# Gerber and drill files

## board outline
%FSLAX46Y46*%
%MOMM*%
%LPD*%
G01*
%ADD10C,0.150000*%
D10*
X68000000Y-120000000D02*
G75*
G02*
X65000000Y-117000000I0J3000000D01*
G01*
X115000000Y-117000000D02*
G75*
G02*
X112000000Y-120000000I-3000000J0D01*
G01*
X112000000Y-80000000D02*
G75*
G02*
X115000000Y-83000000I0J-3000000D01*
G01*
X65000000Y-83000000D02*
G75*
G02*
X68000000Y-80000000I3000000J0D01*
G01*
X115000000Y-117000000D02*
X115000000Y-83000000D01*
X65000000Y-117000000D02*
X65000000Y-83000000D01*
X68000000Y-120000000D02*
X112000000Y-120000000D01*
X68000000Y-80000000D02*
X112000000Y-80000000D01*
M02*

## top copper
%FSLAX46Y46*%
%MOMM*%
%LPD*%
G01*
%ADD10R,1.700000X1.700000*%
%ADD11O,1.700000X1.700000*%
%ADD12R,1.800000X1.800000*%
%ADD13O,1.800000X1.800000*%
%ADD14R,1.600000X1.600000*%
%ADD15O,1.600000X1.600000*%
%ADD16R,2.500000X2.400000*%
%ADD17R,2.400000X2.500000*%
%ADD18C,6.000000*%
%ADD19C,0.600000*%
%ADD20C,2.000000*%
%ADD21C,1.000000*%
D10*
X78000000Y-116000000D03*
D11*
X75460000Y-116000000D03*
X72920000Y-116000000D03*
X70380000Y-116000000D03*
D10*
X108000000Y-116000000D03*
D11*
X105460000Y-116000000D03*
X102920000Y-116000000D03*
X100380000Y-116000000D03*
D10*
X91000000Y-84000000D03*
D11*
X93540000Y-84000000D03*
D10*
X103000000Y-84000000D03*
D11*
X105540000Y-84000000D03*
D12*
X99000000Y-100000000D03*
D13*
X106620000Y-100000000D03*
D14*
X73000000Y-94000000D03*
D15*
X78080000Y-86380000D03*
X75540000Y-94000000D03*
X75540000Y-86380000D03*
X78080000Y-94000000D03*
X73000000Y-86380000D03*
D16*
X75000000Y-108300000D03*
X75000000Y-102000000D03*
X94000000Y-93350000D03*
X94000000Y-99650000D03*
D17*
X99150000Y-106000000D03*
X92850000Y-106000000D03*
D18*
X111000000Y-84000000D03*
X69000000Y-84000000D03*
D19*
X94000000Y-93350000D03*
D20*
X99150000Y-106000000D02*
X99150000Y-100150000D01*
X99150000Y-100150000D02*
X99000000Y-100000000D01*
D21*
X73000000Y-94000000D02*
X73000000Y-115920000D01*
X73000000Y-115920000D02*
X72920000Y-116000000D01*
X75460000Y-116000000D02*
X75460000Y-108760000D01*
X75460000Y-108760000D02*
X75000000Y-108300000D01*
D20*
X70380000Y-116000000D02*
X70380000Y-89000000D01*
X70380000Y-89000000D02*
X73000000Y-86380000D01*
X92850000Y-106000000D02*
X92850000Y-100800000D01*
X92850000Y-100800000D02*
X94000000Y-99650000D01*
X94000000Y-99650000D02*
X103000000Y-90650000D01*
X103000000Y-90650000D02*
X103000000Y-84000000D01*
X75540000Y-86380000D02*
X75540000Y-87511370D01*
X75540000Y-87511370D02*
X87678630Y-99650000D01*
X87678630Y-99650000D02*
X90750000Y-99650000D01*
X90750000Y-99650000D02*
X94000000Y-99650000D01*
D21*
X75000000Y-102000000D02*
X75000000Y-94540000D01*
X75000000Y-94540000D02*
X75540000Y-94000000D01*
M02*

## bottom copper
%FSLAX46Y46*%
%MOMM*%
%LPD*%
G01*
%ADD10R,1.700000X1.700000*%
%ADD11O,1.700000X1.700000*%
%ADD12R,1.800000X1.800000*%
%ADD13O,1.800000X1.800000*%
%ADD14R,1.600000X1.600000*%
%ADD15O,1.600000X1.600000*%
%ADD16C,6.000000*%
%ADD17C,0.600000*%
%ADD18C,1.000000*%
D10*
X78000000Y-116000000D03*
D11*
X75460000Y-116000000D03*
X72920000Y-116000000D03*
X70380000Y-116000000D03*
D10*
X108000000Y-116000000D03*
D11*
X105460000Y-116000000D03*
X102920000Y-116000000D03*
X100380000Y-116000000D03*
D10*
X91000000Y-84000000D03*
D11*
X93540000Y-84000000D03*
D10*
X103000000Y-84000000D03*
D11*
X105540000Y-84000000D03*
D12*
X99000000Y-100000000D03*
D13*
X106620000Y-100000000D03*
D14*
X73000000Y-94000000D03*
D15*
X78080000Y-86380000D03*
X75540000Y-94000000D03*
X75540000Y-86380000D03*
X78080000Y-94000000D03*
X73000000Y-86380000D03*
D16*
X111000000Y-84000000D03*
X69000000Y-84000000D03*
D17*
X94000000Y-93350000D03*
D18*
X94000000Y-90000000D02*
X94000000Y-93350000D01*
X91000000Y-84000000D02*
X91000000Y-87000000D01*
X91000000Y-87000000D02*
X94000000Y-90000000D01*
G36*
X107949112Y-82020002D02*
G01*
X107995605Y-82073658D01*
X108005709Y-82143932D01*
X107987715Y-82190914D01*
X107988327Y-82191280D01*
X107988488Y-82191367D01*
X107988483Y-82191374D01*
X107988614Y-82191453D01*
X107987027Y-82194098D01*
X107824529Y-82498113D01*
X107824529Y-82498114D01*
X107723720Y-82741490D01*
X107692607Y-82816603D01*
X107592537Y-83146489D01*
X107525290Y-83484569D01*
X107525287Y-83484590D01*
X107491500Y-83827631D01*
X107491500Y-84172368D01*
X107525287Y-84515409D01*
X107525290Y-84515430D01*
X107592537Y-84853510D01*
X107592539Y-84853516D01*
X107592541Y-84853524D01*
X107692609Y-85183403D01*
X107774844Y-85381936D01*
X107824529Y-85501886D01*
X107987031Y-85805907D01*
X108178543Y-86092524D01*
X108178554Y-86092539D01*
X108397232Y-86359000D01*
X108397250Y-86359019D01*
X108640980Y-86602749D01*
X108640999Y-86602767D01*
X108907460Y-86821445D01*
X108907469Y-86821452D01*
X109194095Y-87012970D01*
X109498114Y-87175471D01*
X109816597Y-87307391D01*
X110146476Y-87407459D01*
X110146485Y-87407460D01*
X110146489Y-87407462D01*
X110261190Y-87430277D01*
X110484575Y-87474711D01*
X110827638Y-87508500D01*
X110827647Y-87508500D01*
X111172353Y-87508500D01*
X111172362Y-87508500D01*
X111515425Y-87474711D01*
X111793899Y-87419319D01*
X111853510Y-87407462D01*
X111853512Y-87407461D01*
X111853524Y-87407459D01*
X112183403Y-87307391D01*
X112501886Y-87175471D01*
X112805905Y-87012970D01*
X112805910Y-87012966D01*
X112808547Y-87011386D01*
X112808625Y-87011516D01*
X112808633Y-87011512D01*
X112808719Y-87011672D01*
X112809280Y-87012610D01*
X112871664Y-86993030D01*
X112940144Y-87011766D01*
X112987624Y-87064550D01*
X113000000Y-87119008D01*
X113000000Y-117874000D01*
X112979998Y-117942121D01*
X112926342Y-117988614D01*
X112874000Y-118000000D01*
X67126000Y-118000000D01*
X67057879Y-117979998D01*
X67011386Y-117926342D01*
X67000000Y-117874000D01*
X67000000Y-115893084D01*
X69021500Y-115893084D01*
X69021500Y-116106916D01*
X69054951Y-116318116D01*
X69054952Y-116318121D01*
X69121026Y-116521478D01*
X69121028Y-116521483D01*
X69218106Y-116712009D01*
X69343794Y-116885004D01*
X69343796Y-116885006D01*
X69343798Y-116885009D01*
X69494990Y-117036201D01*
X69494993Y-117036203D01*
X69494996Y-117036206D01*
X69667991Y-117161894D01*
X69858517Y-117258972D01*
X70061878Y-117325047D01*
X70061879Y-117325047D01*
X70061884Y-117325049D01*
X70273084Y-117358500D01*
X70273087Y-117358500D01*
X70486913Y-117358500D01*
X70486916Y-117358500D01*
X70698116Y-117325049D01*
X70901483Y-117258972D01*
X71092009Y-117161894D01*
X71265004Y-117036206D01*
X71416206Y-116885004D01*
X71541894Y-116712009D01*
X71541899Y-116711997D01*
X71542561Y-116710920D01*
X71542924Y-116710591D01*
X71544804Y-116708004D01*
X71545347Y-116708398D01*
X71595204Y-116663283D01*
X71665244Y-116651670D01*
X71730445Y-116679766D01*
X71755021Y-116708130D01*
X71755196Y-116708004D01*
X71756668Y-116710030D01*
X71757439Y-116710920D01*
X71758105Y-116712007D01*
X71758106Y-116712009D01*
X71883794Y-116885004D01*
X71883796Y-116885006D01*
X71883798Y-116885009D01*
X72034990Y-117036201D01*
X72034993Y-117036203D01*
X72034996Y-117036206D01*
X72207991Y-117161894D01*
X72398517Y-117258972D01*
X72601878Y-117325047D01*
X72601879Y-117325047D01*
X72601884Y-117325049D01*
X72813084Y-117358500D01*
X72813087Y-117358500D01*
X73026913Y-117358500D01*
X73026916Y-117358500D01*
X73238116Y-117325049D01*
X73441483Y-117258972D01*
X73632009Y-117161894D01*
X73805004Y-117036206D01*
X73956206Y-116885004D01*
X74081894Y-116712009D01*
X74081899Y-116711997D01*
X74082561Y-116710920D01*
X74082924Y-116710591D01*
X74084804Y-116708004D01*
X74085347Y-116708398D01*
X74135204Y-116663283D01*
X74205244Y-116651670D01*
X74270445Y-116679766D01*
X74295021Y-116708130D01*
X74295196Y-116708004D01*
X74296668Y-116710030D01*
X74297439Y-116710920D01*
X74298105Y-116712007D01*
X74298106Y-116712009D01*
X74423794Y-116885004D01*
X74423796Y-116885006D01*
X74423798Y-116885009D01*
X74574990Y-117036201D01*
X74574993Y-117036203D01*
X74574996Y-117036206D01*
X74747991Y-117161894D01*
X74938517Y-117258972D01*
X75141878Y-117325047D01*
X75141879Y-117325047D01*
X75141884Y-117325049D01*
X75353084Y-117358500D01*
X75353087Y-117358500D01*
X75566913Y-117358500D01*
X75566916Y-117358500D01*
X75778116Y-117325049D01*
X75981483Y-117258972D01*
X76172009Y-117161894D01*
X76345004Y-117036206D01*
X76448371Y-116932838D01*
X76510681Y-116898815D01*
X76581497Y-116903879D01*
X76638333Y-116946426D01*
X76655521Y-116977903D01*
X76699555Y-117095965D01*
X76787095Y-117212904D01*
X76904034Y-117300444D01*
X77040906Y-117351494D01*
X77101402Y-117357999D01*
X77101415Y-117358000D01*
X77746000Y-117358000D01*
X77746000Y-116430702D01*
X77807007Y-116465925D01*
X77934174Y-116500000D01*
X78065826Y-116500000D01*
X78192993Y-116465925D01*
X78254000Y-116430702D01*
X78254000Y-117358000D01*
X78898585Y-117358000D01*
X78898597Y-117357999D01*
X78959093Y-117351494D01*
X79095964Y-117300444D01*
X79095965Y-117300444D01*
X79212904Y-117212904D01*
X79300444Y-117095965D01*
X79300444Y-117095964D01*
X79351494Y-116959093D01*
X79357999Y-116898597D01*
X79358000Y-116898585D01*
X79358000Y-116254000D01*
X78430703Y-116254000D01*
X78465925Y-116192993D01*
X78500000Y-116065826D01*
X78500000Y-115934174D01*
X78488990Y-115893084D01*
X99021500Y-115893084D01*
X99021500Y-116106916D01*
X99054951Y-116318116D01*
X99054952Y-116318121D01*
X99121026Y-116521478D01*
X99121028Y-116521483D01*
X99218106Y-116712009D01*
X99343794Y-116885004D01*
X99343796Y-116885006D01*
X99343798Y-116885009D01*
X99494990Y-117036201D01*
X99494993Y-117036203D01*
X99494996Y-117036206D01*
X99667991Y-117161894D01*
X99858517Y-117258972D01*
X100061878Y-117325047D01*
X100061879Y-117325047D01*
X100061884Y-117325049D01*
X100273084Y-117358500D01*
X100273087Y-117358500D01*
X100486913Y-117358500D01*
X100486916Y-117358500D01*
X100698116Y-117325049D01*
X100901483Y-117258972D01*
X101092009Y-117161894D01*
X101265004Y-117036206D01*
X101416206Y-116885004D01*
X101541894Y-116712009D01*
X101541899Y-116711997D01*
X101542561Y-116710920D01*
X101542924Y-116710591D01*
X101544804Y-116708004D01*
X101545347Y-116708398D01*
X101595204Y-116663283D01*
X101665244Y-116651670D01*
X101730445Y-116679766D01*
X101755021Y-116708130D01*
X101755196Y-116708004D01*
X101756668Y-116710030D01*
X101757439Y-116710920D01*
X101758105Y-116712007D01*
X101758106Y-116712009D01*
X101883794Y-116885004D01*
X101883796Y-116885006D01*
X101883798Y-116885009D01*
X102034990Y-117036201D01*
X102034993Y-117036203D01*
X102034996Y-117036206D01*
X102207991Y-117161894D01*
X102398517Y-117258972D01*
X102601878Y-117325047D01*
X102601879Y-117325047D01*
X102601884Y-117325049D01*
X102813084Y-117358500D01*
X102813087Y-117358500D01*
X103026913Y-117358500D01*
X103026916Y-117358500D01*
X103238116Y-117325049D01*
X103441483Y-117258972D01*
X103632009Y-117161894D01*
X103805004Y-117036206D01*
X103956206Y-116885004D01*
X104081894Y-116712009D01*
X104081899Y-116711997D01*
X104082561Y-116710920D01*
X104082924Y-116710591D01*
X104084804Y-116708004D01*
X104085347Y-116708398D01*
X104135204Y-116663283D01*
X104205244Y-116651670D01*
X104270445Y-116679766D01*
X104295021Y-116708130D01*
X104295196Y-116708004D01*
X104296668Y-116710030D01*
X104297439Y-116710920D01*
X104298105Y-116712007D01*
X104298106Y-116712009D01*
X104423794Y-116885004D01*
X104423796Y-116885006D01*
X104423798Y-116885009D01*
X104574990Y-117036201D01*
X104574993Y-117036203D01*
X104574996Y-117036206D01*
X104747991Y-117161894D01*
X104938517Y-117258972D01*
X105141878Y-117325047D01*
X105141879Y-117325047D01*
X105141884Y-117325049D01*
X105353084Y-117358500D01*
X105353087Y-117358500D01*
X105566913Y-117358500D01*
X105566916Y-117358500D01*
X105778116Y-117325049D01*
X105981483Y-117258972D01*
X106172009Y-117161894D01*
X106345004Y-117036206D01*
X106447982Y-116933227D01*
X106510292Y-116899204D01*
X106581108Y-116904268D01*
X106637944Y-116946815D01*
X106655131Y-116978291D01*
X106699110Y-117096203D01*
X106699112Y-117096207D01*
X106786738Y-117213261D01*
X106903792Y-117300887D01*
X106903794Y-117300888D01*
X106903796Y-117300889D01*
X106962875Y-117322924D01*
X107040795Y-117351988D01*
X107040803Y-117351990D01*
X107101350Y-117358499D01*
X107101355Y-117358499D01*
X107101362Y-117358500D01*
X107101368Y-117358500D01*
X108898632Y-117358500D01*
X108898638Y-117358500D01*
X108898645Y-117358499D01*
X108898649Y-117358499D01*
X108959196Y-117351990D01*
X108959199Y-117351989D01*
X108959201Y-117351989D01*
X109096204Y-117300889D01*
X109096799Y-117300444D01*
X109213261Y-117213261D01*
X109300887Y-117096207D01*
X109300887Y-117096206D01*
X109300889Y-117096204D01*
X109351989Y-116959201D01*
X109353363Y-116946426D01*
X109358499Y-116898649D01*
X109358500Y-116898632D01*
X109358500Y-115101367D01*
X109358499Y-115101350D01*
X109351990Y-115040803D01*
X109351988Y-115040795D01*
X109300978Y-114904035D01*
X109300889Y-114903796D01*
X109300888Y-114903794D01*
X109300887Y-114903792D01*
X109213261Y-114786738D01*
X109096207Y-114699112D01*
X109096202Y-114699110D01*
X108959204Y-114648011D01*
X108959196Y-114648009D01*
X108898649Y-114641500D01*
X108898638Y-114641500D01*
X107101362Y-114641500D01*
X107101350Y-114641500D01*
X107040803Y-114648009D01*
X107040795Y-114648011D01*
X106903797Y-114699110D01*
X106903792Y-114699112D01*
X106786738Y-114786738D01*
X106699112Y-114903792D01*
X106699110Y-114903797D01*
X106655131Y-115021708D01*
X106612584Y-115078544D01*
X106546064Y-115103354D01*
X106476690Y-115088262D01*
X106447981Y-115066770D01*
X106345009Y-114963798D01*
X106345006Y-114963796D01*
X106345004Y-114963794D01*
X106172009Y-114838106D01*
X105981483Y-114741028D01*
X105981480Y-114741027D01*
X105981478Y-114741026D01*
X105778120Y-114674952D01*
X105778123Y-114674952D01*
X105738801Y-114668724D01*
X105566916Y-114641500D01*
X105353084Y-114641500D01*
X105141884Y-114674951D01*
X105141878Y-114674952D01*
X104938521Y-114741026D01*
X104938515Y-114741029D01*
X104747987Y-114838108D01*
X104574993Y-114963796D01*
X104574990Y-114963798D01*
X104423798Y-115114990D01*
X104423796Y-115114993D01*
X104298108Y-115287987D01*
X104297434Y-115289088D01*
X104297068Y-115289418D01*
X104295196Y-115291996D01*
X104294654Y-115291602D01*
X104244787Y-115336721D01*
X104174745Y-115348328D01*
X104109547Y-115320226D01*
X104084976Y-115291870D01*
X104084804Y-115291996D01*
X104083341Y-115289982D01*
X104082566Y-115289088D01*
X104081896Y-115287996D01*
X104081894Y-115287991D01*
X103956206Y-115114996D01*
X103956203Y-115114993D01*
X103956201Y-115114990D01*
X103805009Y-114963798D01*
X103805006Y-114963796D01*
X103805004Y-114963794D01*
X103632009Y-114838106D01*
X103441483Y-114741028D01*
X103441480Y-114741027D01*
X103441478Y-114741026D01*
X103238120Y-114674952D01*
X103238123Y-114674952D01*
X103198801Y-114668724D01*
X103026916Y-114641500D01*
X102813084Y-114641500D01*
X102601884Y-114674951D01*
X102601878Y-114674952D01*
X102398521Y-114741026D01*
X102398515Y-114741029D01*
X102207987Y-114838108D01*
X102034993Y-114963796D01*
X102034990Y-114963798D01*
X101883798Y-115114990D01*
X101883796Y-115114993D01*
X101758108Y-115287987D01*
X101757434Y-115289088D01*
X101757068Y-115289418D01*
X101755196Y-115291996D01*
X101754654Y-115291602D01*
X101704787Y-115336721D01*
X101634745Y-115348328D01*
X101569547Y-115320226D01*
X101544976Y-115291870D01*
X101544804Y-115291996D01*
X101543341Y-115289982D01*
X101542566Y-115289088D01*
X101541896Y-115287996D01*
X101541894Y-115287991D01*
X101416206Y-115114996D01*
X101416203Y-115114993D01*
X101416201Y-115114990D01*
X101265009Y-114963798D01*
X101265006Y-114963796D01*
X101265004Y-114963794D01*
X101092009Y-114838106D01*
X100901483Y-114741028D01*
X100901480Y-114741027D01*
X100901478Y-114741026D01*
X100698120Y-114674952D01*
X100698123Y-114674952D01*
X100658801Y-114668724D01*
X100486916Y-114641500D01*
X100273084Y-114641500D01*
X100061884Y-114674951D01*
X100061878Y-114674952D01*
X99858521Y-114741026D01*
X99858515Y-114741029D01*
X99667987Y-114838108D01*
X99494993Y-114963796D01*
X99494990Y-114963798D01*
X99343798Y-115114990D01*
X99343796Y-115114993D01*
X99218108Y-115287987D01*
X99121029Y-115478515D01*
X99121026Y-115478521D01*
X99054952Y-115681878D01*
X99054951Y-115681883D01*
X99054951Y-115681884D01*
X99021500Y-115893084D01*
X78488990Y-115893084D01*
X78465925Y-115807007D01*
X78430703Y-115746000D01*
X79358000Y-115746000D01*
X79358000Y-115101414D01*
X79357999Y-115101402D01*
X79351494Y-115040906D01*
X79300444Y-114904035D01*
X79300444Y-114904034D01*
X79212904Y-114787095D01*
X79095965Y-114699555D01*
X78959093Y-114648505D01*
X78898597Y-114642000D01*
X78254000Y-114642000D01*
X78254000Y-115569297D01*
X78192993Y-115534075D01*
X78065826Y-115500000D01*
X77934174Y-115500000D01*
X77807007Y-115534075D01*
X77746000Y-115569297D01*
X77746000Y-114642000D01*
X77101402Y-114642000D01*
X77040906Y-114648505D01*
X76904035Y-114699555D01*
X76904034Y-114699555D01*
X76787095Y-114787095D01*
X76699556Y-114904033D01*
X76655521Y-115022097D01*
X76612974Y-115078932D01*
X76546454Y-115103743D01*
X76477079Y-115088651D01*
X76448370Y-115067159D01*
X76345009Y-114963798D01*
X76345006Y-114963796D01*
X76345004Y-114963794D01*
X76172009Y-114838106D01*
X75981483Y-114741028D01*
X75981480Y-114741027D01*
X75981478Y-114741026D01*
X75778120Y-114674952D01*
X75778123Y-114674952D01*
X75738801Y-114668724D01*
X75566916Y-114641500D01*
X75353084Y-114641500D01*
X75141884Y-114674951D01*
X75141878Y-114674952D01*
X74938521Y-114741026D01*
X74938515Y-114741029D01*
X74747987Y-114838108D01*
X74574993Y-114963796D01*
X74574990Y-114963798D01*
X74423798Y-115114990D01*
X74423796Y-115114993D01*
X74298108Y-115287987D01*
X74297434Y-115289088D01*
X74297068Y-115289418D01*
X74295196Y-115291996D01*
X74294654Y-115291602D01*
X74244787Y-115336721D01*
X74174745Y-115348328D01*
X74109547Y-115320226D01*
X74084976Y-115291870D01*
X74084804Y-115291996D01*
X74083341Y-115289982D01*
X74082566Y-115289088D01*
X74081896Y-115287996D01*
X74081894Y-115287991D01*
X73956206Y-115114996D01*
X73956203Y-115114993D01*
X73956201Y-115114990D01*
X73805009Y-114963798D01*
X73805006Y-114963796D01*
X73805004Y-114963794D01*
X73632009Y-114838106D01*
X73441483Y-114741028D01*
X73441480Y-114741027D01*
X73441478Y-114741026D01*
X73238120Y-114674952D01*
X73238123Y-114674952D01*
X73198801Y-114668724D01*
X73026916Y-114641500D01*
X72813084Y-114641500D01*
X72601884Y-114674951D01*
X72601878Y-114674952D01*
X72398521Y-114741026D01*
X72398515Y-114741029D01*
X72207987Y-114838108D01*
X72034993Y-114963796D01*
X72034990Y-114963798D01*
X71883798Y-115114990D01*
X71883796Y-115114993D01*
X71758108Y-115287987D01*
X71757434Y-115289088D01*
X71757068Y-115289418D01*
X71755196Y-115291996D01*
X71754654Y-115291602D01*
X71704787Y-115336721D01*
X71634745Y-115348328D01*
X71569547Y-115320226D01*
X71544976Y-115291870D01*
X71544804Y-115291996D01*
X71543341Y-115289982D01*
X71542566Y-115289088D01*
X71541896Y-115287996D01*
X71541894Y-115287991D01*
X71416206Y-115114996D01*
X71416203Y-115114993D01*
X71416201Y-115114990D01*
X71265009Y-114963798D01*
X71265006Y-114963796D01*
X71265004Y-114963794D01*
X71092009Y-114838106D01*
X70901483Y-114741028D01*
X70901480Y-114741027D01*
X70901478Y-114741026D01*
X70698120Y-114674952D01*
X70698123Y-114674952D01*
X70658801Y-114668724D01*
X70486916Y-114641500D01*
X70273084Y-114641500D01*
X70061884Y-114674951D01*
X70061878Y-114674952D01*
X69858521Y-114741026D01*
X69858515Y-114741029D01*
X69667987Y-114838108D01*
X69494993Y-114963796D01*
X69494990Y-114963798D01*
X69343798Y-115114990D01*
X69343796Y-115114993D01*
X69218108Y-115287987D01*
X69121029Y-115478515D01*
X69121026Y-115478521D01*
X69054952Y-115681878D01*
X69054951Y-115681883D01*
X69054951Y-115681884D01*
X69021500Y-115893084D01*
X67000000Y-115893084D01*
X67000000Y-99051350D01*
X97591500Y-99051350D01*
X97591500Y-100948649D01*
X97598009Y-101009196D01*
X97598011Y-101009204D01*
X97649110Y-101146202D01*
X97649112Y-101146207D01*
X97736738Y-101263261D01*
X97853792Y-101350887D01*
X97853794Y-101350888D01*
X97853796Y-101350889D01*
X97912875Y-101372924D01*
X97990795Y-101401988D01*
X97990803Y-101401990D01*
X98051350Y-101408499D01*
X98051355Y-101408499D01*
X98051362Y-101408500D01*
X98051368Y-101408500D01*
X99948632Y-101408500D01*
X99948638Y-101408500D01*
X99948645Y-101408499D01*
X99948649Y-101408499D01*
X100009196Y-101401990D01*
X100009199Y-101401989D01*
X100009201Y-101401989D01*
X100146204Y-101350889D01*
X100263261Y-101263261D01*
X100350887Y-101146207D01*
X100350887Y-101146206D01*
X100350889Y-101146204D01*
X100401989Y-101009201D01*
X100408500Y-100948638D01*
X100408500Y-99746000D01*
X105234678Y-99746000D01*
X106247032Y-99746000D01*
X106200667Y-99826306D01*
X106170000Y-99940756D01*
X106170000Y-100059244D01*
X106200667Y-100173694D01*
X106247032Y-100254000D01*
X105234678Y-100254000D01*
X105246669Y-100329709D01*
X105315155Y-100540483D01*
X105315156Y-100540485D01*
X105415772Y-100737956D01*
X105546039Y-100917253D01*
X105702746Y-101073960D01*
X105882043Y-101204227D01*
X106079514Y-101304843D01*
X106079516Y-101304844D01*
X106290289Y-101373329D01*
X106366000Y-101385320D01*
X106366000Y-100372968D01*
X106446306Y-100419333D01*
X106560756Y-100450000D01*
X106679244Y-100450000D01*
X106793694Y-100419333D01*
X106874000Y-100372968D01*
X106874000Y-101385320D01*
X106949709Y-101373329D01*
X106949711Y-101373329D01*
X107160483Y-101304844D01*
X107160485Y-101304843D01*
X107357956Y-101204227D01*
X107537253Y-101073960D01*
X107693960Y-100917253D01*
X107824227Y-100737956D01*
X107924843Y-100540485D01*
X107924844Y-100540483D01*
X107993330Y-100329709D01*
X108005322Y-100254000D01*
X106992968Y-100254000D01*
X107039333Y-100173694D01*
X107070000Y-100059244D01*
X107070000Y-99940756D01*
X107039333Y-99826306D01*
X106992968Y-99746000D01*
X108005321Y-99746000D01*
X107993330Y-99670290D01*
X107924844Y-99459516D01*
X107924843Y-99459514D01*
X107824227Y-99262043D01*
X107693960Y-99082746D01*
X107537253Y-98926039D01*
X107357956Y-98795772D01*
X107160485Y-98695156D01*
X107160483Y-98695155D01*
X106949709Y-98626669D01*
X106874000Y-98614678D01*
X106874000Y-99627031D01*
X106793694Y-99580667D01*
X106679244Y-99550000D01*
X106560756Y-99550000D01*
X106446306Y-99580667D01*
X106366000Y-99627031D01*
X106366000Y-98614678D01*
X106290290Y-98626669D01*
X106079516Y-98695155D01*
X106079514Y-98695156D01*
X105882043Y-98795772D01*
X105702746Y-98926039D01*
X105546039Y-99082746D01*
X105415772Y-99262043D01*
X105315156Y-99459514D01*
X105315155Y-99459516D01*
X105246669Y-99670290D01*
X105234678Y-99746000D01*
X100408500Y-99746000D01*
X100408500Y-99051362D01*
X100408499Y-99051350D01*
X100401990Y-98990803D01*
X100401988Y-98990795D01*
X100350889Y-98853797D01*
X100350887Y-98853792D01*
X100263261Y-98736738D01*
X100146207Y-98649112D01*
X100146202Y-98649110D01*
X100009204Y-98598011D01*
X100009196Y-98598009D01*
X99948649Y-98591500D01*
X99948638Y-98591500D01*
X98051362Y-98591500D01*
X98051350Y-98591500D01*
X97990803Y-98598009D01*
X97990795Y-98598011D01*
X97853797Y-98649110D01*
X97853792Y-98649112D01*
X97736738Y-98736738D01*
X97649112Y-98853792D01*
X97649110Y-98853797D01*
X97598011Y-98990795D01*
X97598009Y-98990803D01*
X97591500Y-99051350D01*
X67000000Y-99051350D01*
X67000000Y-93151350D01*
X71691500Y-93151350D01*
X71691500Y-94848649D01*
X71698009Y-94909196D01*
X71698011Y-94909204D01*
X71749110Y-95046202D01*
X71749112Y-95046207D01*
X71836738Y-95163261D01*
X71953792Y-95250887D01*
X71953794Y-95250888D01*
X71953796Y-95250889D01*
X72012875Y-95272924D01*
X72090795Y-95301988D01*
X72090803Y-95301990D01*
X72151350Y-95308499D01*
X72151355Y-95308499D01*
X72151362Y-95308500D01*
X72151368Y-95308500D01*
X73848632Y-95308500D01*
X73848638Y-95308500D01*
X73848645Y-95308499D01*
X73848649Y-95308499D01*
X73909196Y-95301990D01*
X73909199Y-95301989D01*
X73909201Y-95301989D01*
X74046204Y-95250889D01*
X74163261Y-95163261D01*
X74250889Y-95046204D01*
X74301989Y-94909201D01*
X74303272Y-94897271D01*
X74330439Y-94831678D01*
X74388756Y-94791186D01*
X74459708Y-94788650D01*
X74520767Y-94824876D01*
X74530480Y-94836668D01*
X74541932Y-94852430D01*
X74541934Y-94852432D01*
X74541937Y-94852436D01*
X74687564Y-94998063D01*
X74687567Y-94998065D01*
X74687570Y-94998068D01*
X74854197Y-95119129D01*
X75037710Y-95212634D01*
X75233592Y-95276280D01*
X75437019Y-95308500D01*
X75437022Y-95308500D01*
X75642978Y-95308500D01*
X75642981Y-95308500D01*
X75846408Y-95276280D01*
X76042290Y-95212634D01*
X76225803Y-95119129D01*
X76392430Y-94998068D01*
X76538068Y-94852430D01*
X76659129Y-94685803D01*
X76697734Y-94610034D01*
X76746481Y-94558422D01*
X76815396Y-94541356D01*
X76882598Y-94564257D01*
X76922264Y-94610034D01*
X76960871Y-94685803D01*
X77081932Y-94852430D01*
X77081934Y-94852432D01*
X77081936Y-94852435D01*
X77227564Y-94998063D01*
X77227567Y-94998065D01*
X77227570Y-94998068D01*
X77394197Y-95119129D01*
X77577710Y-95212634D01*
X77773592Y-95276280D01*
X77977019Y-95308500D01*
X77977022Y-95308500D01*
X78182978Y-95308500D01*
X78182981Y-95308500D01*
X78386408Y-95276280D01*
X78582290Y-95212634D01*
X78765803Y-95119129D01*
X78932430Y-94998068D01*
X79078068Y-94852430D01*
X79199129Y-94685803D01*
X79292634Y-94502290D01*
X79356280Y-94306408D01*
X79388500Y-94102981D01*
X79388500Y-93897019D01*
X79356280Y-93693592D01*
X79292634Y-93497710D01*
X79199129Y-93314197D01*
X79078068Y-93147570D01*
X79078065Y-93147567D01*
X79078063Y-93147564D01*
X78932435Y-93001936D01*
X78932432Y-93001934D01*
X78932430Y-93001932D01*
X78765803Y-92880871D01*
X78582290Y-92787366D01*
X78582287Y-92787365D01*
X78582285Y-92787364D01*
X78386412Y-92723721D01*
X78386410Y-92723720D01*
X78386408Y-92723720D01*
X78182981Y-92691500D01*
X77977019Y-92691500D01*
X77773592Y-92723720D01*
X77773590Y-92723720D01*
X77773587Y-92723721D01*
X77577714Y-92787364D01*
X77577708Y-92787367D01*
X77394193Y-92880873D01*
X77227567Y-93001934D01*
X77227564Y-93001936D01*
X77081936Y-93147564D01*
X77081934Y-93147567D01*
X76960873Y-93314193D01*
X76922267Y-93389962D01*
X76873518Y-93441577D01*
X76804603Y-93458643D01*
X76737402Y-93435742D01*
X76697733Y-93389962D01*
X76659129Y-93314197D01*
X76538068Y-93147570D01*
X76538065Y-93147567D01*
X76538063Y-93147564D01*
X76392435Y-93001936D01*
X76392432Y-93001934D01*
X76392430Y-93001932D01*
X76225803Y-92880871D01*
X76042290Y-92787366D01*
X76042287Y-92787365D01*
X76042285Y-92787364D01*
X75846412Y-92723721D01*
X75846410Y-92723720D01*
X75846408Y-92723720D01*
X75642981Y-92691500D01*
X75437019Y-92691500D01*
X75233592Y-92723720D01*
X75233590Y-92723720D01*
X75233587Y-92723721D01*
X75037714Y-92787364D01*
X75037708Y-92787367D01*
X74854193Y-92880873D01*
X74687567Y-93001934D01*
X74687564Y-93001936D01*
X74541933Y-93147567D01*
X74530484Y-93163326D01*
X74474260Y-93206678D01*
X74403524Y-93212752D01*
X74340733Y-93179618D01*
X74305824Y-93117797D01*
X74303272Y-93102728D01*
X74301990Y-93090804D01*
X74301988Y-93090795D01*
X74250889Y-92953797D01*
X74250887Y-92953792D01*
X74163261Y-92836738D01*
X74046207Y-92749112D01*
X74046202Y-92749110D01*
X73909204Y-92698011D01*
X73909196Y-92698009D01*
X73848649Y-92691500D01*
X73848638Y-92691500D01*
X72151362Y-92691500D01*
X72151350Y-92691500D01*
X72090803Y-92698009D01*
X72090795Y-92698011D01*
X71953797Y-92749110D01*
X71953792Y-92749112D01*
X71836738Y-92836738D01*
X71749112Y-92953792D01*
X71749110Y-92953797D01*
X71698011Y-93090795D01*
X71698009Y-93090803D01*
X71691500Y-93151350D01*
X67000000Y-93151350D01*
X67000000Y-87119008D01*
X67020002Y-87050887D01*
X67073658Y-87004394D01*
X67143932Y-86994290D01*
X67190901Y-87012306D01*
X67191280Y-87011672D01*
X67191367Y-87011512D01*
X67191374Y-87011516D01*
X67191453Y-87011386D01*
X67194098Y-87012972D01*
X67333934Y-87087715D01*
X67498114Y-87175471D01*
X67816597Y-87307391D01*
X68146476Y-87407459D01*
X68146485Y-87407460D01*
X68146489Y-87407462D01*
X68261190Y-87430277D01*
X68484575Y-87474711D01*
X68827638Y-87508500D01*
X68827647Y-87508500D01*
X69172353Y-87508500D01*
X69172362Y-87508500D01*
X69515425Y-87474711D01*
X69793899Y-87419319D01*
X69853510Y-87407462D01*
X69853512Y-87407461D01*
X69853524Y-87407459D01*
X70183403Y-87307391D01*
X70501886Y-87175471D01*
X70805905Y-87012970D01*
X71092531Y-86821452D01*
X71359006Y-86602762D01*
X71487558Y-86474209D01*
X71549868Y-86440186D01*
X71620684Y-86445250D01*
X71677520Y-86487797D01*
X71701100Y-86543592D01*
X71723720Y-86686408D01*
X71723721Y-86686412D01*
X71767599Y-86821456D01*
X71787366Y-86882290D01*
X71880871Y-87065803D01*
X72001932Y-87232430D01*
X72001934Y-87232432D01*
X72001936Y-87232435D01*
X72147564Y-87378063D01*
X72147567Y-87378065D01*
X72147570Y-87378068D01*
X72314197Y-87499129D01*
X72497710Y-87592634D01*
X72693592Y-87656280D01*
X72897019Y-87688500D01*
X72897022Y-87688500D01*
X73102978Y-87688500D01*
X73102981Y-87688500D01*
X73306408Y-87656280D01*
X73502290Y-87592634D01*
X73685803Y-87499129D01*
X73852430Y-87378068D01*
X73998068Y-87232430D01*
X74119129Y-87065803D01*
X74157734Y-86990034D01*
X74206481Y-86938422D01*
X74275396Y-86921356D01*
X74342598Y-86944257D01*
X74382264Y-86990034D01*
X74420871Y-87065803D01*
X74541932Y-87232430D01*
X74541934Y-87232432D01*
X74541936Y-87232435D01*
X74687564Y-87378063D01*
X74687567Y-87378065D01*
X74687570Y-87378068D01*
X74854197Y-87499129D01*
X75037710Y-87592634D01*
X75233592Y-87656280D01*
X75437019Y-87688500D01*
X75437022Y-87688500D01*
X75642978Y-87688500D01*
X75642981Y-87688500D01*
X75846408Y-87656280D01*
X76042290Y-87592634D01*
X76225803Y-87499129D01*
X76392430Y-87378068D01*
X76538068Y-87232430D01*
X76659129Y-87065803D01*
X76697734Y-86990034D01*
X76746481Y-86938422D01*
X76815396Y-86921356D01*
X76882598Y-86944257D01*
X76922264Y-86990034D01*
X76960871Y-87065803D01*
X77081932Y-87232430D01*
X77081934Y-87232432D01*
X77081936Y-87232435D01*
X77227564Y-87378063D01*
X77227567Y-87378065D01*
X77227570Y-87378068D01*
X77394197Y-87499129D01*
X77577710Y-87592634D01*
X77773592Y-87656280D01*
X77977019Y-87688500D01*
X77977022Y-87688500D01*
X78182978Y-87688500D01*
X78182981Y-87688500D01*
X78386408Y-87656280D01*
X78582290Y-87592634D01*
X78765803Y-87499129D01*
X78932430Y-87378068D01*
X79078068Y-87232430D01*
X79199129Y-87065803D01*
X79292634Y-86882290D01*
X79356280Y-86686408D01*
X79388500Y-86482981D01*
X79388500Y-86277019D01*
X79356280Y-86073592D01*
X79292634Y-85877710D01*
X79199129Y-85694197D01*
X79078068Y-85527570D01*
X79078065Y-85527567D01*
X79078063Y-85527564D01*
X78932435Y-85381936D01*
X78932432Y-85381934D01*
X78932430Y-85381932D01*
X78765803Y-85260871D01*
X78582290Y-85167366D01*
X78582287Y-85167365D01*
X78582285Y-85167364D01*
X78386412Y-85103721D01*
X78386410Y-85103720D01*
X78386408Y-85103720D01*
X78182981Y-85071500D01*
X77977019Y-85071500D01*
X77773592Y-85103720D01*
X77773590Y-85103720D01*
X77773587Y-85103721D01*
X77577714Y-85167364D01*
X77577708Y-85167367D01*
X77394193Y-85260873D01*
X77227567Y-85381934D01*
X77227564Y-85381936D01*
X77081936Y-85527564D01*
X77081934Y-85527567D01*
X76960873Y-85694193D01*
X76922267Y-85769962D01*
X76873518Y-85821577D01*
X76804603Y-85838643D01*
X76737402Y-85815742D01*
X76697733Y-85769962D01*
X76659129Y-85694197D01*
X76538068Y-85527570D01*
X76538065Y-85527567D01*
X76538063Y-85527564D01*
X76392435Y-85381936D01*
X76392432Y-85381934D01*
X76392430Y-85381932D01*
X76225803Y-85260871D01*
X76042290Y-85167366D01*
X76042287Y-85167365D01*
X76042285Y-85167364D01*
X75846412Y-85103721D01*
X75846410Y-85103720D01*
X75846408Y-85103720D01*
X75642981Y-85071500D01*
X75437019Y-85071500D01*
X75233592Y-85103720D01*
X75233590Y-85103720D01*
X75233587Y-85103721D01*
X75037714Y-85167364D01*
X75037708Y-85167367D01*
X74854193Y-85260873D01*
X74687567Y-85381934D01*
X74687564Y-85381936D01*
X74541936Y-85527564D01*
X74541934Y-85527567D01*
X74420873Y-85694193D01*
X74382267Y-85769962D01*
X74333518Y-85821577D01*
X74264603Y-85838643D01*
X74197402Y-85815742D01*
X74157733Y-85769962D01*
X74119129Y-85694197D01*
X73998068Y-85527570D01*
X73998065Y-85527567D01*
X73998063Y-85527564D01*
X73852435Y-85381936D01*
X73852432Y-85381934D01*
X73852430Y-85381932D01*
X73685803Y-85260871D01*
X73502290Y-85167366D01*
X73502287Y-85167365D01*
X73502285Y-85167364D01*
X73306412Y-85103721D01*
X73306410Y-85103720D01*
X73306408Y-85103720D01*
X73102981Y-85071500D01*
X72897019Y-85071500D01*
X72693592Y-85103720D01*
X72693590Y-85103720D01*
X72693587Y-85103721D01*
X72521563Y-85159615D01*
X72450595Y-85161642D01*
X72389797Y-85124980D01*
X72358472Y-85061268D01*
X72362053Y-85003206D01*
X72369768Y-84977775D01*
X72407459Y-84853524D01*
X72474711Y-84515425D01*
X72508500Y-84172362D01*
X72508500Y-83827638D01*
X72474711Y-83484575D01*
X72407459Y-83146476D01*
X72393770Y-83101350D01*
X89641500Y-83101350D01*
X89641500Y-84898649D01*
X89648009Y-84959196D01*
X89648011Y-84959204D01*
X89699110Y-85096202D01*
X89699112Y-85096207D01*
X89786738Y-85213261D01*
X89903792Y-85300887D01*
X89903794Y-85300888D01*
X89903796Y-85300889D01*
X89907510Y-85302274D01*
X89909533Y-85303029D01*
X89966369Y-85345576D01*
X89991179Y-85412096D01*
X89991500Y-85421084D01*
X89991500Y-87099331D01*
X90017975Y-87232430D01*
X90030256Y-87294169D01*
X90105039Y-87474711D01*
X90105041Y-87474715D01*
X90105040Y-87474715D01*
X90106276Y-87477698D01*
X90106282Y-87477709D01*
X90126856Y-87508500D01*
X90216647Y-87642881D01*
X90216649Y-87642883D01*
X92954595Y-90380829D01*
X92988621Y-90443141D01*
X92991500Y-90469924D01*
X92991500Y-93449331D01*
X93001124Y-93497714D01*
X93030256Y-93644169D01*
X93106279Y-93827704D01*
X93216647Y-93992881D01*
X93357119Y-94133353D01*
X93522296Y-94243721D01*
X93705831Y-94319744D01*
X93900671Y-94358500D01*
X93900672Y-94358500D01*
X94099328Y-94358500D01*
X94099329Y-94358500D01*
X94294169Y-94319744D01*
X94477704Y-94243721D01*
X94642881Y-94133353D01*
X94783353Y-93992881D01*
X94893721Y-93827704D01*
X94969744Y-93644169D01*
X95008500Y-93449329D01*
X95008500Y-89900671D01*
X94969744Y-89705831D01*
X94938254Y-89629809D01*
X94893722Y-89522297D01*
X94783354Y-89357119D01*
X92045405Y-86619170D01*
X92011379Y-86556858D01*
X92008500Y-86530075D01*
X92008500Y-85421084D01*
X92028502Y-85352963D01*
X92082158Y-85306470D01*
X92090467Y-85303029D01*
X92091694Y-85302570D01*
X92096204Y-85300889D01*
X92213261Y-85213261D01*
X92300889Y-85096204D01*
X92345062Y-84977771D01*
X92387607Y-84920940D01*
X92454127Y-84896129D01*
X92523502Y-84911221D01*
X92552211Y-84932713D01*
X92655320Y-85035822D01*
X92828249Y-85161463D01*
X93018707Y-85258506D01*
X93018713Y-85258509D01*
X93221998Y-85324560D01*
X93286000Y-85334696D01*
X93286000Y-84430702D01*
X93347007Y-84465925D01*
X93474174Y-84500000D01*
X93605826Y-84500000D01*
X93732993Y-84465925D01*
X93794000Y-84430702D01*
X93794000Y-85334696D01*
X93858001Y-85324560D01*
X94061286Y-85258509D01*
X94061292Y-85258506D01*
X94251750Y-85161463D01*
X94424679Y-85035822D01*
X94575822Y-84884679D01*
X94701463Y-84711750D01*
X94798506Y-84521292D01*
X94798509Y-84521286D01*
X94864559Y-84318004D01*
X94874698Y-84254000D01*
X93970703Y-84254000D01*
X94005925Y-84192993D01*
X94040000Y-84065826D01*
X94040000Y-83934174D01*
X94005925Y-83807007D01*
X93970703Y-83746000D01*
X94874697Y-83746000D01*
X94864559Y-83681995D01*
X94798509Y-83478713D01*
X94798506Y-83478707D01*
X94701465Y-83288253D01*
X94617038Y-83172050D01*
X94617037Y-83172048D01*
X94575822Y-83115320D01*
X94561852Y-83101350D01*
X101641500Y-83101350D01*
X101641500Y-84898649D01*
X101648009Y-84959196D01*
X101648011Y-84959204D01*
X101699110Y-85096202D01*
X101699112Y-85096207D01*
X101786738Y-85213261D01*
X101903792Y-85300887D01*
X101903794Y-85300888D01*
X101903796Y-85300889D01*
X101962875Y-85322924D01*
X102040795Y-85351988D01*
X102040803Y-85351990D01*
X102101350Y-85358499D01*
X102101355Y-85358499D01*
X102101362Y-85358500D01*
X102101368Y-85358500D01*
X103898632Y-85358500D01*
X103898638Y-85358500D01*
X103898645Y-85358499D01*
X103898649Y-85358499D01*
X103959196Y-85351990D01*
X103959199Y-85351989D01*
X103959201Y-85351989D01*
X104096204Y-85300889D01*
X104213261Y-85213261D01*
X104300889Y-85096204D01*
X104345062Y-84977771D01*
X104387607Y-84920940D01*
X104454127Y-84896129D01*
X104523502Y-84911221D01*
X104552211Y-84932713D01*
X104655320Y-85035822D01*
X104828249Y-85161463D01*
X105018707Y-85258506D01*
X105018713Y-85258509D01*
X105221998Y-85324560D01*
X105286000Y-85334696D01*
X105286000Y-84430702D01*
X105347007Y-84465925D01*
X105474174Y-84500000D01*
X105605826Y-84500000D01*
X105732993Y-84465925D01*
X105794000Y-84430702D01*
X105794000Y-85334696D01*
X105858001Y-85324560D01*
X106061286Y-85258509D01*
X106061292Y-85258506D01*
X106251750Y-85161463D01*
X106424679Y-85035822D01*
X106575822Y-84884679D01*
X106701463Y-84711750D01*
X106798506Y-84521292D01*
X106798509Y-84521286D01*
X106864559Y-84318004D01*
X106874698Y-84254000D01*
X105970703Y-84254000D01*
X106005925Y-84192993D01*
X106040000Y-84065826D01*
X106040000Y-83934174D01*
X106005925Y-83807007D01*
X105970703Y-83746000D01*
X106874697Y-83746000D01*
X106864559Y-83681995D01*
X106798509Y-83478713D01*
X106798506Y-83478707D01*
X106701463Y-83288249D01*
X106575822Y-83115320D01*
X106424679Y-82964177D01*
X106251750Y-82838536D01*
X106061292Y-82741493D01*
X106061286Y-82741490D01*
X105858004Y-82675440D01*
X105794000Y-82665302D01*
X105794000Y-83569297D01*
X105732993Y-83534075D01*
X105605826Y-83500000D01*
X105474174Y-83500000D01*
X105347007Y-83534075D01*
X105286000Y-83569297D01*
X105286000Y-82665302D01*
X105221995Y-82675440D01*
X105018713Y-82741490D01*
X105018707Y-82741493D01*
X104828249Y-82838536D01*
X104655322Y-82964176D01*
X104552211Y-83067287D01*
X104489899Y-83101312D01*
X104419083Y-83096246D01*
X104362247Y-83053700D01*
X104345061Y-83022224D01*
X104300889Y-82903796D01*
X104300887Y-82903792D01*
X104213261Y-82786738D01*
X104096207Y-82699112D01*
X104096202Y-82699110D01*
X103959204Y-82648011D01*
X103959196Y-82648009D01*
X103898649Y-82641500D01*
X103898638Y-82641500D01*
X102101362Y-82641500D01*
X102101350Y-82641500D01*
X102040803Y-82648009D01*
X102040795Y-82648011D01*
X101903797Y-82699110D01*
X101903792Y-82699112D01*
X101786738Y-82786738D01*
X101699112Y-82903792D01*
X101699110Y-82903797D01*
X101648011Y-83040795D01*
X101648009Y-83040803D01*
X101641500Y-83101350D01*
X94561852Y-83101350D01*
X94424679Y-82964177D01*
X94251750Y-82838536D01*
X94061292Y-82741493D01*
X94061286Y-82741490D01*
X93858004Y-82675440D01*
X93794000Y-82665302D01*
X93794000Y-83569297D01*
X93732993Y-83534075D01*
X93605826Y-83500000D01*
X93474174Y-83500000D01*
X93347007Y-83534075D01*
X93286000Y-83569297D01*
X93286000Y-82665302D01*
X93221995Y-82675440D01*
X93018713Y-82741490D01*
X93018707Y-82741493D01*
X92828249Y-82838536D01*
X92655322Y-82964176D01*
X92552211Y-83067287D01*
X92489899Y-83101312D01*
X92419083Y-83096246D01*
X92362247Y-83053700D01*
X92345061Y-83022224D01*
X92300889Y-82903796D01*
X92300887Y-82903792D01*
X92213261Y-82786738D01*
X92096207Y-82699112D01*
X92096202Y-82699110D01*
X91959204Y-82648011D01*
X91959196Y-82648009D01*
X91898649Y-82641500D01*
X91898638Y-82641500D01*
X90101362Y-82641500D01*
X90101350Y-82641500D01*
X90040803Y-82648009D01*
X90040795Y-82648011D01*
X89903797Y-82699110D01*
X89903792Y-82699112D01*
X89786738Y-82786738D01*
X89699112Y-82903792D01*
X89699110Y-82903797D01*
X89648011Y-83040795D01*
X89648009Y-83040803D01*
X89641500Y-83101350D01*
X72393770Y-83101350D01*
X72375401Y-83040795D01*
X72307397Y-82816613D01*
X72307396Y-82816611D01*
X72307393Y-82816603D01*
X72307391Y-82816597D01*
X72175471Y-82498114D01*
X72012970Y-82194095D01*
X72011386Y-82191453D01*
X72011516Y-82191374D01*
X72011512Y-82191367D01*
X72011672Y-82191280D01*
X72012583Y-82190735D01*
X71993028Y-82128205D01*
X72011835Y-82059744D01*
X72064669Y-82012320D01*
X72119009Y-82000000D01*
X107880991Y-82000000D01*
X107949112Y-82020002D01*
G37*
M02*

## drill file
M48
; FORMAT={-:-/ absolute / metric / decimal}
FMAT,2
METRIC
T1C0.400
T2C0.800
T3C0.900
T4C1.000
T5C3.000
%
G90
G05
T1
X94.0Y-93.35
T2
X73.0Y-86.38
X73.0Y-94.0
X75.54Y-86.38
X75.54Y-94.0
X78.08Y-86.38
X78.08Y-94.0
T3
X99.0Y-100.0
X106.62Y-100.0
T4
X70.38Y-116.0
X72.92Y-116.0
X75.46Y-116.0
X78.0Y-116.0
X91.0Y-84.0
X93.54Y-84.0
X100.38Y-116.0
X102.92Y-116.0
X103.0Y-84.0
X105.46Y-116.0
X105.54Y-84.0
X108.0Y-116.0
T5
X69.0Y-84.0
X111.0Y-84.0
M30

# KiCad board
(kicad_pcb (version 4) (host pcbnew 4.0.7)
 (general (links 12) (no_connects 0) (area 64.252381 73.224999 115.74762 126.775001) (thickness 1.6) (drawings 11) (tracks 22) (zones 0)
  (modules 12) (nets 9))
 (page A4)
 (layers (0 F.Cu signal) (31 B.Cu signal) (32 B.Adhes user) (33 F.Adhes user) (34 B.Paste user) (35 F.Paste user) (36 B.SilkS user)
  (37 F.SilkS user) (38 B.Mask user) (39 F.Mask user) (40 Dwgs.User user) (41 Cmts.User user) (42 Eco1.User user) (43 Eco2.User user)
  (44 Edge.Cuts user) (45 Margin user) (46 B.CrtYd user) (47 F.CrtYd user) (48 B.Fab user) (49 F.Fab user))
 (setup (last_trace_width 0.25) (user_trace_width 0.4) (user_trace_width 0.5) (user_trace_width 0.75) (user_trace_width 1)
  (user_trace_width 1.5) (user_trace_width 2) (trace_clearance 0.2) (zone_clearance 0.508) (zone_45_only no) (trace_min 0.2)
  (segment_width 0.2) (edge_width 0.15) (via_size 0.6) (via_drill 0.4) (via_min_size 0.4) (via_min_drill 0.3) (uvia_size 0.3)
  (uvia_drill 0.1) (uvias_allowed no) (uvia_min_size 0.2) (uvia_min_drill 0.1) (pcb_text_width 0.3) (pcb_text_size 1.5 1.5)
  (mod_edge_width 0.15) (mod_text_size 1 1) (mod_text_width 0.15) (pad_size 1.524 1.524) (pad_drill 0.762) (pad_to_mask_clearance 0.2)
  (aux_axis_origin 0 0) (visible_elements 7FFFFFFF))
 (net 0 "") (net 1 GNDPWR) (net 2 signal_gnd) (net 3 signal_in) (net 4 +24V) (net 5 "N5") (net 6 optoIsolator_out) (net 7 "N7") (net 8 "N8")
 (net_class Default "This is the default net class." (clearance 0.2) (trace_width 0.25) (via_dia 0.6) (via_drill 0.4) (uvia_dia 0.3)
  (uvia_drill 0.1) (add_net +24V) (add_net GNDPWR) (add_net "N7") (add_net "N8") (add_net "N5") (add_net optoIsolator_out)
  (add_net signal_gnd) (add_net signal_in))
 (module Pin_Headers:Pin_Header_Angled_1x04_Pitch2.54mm (layer F.Cu) (at 78 116 270)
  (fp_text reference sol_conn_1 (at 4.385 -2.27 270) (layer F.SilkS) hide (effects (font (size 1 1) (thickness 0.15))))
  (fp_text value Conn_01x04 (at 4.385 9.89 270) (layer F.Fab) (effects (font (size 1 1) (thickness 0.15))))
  (pad 1 thru_hole rect (at 0 0 270) (size 1.7 1.7) (drill 1) (layers *.Cu *.Mask) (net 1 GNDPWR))
  (pad 2 thru_hole oval (at 0 2.54 270) (size 1.7 1.7) (drill 1) (layers *.Cu *.Mask) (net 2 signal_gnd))
  (pad 3 thru_hole oval (at 0 5.08 270) (size 1.7 1.7) (drill 1) (layers *.Cu *.Mask) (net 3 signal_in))
  (pad 4 thru_hole oval (at 0 7.62 270) (size 1.7 1.7) (drill 1) (layers *.Cu *.Mask) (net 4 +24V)))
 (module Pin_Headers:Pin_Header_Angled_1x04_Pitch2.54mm (layer F.Cu) (at 108 116 270)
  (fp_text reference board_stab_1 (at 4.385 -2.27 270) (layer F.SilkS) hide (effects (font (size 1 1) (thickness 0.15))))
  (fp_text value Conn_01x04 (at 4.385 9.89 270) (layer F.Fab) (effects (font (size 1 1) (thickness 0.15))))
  (pad 1 thru_hole rect (at 0 0 270) (size 1.7 1.7) (drill 1) (layers *.Cu *.Mask))
  (pad 2 thru_hole oval (at 0 2.54 270) (size 1.7 1.7) (drill 1) (layers *.Cu *.Mask))
  (pad 3 thru_hole oval (at 0 5.08 270) (size 1.7 1.7) (drill 1) (layers *.Cu *.Mask))
  (pad 4 thru_hole oval (at 0 7.62 270) (size 1.7 1.7) (drill 1) (layers *.Cu *.Mask)))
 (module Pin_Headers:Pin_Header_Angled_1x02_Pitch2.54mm (layer F.Cu) (at 91 84 90)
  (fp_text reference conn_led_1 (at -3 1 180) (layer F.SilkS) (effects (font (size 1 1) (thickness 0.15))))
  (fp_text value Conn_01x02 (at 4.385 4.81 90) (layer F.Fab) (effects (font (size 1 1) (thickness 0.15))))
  (pad 1 thru_hole rect (at 0 0 90) (size 1.7 1.7) (drill 1) (layers *.Cu *.Mask) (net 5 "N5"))
  (pad 2 thru_hole oval (at 0 2.54 90) (size 1.7 1.7) (drill 1) (layers *.Cu *.Mask) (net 1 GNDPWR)))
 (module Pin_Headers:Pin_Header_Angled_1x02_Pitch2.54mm (layer F.Cu) (at 103 84 90)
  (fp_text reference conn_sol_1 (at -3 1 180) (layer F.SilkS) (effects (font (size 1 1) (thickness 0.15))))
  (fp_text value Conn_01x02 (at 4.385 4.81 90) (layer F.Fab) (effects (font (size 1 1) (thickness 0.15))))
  (pad 1 thru_hole rect (at 0 0 90) (size 1.7 1.7) (drill 1) (layers *.Cu *.Mask) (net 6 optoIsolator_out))
  (pad 2 thru_hole oval (at 0 2.54 90) (size 1.7 1.7) (drill 1) (layers *.Cu *.Mask) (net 1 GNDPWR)))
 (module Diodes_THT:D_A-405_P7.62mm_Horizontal (layer F.Cu) (at 99 100)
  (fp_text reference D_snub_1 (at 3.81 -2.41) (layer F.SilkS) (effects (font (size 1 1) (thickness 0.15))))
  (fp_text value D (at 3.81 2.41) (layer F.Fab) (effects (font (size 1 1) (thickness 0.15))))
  (pad 1 thru_hole rect (at 0 0) (size 1.8 1.8) (drill 0.9) (layers *.Cu *.Mask) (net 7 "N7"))
  (pad 2 thru_hole oval (at 7.62 0) (size 1.8 1.8) (drill 0.9) (layers *.Cu *.Mask) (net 1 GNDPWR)))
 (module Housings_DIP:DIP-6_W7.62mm (layer F.Cu) (at 73 94 90)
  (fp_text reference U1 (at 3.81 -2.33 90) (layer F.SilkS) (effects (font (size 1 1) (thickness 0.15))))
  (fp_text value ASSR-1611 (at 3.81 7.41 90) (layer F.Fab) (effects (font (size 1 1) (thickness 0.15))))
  (pad 1 thru_hole rect (at 0 0 90) (size 1.6 1.6) (drill 0.8) (layers *.Cu *.Mask) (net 3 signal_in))
  (pad 4 thru_hole oval (at 7.62 5.08 90) (size 1.6 1.6) (drill 0.8) (layers *.Cu *.Mask))
  (pad 2 thru_hole oval (at 0 2.54 90) (size 1.6 1.6) (drill 0.8) (layers *.Cu *.Mask) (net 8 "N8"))
  (pad 5 thru_hole oval (at 7.62 2.54 90) (size 1.6 1.6) (drill 0.8) (layers *.Cu *.Mask) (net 6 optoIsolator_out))
  (pad 3 thru_hole oval (at 0 5.08 90) (size 1.6 1.6) (drill 0.8) (layers *.Cu *.Mask))
  (pad 6 thru_hole oval (at 7.62 0 90) (size 1.6 1.6) (drill 0.8) (layers *.Cu *.Mask) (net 4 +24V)))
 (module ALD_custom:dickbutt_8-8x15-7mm (layer F.Cu) (at 81 103.5)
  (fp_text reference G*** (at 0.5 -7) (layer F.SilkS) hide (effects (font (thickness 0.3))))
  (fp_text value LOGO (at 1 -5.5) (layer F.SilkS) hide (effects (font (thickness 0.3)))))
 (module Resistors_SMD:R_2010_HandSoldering (layer F.Cu) (at 75 105.15 90)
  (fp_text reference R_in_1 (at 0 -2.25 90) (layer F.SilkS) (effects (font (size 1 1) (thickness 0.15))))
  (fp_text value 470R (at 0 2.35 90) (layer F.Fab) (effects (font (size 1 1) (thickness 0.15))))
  (pad 1 smd rect (at -3.15 0 90) (size 2.4 2.5) (layers F.Cu F.Paste F.Mask) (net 2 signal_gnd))
  (pad 2 smd rect (at 3.15 0 90) (size 2.4 2.5) (layers F.Cu F.Paste F.Mask) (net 8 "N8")))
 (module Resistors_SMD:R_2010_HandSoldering (layer F.Cu) (at 94 96.5 270)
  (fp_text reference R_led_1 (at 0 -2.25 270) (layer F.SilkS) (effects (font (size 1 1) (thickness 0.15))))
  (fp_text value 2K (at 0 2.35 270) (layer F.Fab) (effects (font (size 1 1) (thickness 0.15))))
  (pad 1 smd rect (at -3.15 0 270) (size 2.4 2.5) (layers F.Cu F.Paste F.Mask) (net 5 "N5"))
  (pad 2 smd rect (at 3.15 0 270) (size 2.4 2.5) (layers F.Cu F.Paste F.Mask) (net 6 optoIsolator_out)))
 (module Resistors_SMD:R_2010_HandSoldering (layer F.Cu) (at 96 106 180)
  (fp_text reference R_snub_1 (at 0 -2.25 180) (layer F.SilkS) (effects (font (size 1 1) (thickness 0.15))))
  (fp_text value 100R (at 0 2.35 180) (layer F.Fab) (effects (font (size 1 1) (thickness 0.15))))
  (pad 1 smd rect (at -3.15 0 180) (size 2.4 2.5) (layers F.Cu F.Paste F.Mask) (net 7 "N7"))
  (pad 2 smd rect (at 3.15 0 180) (size 2.4 2.5) (layers F.Cu F.Paste F.Mask) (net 6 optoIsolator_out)))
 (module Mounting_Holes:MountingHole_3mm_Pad (layer F.Cu) (at 111 84)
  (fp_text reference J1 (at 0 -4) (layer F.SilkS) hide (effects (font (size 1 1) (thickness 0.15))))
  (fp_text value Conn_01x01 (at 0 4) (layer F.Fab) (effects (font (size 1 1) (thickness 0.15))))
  (pad 1 thru_hole circle (at 0 0) (size 6 6) (drill 3) (layers *.Cu *.Mask)))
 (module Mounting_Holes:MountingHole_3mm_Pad (layer F.Cu) (at 69 84)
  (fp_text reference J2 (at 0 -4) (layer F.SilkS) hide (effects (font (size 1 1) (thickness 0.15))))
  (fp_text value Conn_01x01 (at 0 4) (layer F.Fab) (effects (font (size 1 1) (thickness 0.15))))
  (pad 1 thru_hole circle (at 0 0) (size 6 6) (drill 3) (layers *.Cu *.Mask)))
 (gr_arc (start 68 117) (end 68 120) (angle 90) (layer Edge.Cuts) (width 0.15))
 (gr_arc (start 112 117) (end 115 117) (angle 90) (layer Edge.Cuts) (width 0.15))
 (gr_arc (start 112 83) (end 112 80) (angle 90) (layer Edge.Cuts) (width 0.15))
 (gr_arc (start 68 83) (end 65 83) (angle 90) (layer Edge.Cuts) (width 0.15))
 (gr_line (start 115 117) (end 115 83) (angle 90) (layer Edge.Cuts) (width 0.15))
 (gr_line (start 65 117) (end 65 83) (angle 90) (layer Edge.Cuts) (width 0.15))
 (gr_line (start 68 120) (end 112 120) (angle 90) (layer Edge.Cuts) (width 0.15))
 (gr_line (start 68 80) (end 112 80) (angle 90) (layer Edge.Cuts) (width 0.15))
 (segment (start 94 90) (end 94 93.35) (width 1) (layer B.Cu) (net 5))
 (via (at 94 93.35) (size 0.6) (drill 0.4) (layers F.Cu B.Cu) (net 5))
 (segment (start 91 84) (end 91 87) (width 1) (layer B.Cu) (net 5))
 (segment (start 91 87) (end 94 90) (width 1) (layer B.Cu) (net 5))
 (segment (start 99.15 106) (end 99.15 100.15) (width 2) (layer F.Cu) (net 7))
 (segment (start 99.15 100.15) (end 99 100) (width 2) (layer F.Cu) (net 7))
 (segment (start 73 94) (end 73 115.92) (width 1) (layer F.Cu) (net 3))
 (segment (start 73 115.92) (end 72.92 116) (width 1) (layer F.Cu) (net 3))
 (segment (start 75.46 116) (end 75.46 108.76) (width 1) (layer F.Cu) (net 2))
 (segment (start 75.46 108.76) (end 75 108.3) (width 1) (layer F.Cu) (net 2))
 (segment (start 70.38 116) (end 70.38 89) (width 2) (layer F.Cu) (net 4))
 (segment (start 70.38 89) (end 73 86.38) (width 2) (layer F.Cu) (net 4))
 (segment (start 92.85 106) (end 92.85 100.8) (width 2) (layer F.Cu) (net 6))
 (segment (start 92.85 100.8) (end 94 99.65) (width 2) (layer F.Cu) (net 6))
 (segment (start 94 99.65) (end 103 90.65) (width 2) (layer F.Cu) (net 6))
 (segment (start 103 90.65) (end 103 84) (width 2) (layer F.Cu) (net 6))
 (segment (start 75.54 86.38) (end 75.54 87.51137) (width 2) (layer F.Cu) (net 6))
 (segment (start 75.54 87.51137) (end 87.67863 99.65) (width 2) (layer F.Cu) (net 6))
 (segment (start 87.67863 99.65) (end 90.75 99.65) (width 2) (layer F.Cu) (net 6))
 (segment (start 90.75 99.65) (end 94 99.65) (width 2) (layer F.Cu) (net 6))
 (segment (start 75 102) (end 75 94.54) (width 1) (layer F.Cu) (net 8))
 (segment (start 75 94.54) (end 75.54 94) (width 1) (layer F.Cu) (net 8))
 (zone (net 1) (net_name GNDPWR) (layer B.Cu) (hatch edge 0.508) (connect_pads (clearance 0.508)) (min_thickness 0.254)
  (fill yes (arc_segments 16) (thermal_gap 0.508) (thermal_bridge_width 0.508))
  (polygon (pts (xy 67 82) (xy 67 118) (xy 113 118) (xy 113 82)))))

